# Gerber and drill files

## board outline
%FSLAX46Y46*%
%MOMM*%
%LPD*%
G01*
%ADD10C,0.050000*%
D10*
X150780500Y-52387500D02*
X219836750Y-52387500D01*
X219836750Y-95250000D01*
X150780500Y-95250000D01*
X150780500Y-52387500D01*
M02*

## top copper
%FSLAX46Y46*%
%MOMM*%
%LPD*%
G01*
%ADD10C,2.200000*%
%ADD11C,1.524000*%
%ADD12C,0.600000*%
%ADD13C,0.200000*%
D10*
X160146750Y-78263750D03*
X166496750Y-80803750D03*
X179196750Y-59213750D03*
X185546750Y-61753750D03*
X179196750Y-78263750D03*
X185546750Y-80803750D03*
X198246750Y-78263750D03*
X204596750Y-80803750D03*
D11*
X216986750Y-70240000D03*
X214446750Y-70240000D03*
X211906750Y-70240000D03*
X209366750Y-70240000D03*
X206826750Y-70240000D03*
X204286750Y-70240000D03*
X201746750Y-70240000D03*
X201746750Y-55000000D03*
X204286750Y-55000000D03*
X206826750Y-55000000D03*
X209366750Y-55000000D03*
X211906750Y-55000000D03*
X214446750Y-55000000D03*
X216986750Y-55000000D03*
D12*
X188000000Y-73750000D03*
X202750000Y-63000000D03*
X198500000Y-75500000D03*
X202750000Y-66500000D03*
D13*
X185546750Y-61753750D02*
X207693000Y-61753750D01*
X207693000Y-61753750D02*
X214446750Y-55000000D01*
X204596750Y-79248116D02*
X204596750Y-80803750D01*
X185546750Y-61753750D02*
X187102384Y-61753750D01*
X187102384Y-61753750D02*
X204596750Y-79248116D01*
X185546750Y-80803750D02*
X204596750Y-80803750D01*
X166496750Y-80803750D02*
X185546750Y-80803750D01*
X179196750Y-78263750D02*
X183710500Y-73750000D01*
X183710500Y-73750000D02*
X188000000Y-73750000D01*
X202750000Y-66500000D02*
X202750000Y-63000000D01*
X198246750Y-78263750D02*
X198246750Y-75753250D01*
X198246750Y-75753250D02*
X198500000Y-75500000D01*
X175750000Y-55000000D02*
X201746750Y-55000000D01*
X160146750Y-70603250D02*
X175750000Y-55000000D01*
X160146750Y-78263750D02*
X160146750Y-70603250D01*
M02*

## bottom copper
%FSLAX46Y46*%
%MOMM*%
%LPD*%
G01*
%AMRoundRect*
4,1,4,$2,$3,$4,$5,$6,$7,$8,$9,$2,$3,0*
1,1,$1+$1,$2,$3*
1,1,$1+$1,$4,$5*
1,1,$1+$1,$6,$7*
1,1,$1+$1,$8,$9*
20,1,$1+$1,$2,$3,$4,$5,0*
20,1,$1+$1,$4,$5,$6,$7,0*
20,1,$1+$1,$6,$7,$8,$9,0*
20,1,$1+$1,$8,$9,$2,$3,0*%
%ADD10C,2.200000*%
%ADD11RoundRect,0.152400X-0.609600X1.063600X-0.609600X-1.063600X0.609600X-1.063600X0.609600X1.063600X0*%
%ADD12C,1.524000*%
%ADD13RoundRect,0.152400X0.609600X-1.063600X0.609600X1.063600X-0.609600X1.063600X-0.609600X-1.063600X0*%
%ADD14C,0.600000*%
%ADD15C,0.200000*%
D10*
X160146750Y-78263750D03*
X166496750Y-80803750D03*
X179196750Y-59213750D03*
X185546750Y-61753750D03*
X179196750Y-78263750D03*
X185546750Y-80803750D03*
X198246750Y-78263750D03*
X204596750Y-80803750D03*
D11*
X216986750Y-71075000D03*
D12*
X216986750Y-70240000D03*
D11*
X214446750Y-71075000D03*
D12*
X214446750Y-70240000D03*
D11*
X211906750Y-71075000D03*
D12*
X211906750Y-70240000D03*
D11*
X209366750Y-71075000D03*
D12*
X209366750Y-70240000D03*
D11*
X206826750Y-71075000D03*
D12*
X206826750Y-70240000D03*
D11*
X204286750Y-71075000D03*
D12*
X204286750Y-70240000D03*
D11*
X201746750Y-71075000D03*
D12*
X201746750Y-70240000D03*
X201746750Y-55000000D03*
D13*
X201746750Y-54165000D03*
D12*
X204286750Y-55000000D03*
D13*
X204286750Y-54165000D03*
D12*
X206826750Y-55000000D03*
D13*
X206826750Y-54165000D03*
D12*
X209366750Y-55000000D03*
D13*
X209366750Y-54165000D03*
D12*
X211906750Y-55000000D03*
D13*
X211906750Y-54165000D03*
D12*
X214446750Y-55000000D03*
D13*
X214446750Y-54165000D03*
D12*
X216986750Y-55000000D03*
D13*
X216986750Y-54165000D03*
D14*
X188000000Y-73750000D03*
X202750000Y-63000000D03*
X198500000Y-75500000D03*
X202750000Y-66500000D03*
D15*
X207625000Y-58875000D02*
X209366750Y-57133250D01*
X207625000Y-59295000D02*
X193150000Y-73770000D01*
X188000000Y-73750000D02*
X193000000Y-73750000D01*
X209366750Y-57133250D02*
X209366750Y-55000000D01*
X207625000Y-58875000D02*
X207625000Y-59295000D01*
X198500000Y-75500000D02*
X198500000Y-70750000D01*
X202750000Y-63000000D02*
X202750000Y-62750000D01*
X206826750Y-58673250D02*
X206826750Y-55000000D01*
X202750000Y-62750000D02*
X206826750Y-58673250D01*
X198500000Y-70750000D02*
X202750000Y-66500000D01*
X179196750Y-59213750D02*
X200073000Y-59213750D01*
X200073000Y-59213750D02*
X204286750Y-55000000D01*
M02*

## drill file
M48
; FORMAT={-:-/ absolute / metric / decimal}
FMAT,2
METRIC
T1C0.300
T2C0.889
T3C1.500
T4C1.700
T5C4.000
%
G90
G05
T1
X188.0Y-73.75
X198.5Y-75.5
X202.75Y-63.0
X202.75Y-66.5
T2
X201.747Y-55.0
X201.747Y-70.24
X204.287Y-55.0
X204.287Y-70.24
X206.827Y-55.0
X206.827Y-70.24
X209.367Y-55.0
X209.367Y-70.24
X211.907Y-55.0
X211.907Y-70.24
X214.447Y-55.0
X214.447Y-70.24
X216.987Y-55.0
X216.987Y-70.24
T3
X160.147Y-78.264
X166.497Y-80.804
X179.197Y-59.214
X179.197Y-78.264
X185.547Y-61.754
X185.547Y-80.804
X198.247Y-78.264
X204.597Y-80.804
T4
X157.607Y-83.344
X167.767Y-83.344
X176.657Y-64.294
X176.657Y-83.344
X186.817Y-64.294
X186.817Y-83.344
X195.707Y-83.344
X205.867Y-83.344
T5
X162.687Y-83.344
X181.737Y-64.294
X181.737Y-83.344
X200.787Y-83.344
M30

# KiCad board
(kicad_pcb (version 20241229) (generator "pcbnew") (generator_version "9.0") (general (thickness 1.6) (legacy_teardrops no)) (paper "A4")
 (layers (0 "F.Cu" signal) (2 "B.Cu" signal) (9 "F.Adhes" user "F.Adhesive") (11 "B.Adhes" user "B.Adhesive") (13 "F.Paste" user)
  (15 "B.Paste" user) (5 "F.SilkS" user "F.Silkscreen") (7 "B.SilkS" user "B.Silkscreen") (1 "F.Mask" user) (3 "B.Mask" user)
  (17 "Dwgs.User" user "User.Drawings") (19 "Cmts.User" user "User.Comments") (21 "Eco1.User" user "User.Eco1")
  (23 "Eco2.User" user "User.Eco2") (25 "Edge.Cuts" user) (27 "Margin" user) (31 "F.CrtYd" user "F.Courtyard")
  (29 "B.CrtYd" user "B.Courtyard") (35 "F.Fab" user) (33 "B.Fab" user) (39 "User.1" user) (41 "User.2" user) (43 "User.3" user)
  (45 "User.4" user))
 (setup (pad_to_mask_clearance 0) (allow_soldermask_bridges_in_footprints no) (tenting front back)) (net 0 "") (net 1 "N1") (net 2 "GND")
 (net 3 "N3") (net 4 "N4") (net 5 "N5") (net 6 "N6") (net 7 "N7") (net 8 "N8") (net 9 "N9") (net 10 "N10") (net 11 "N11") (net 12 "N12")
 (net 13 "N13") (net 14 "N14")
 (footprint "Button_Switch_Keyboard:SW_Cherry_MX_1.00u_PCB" (layer "B.Cu") (at 160.14675 78.26375 180)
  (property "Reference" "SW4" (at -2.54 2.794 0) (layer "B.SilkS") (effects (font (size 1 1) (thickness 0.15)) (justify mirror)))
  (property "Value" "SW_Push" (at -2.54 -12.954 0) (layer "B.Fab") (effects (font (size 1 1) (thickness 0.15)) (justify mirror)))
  (pad "" np_thru_hole circle (at -7.62 -5.08 180) (size 1.7 1.7) (drill 1.7) (layers "*.Cu" "*.Mask"))
  (pad "" np_thru_hole circle (at -2.54 -5.08 180) (size 4 4) (drill 4) (layers "*.Cu" "*.Mask"))
  (pad "" np_thru_hole circle (at 2.54 -5.08 180) (size 1.7 1.7) (drill 1.7) (layers "*.Cu" "*.Mask"))
  (pad "1" thru_hole circle (at 0 0 180) (size 2.2 2.2) (drill 1.5) (layers "*.Cu" "*.Mask") (remove_unused_layers no) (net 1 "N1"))
  (pad "2" thru_hole circle (at -6.35 -2.54 180) (size 2.2 2.2) (drill 1.5) (layers "*.Cu" "*.Mask") (remove_unused_layers no) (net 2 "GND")))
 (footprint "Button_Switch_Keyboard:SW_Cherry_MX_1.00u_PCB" (layer "B.Cu") (at 179.19675 59.21375 180)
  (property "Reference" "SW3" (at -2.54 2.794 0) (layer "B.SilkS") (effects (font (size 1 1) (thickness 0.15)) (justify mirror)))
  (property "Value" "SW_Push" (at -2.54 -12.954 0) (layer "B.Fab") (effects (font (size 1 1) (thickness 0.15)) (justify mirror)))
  (pad "" np_thru_hole circle (at -7.62 -5.08 180) (size 1.7 1.7) (drill 1.7) (layers "*.Cu" "*.Mask"))
  (pad "" np_thru_hole circle (at -2.54 -5.08 180) (size 4 4) (drill 4) (layers "*.Cu" "*.Mask"))
  (pad "" np_thru_hole circle (at 2.54 -5.08 180) (size 1.7 1.7) (drill 1.7) (layers "*.Cu" "*.Mask"))
  (pad "1" thru_hole circle (at 0 0 180) (size 2.2 2.2) (drill 1.5) (layers "*.Cu" "*.Mask") (remove_unused_layers no) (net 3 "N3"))
  (pad "2" thru_hole circle (at -6.35 -2.54 180) (size 2.2 2.2) (drill 1.5) (layers "*.Cu" "*.Mask") (remove_unused_layers no) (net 2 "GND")))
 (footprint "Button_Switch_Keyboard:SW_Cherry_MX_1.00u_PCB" (layer "B.Cu") (at 179.19675 78.26375 180)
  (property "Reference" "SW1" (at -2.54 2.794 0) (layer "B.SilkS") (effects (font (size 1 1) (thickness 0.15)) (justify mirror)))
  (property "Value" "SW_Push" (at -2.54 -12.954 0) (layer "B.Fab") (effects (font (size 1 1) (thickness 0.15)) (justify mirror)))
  (pad "" np_thru_hole circle (at -7.62 -5.08 180) (size 1.7 1.7) (drill 1.7) (layers "*.Cu" "*.Mask"))
  (pad "" np_thru_hole circle (at -2.54 -5.08 180) (size 4 4) (drill 4) (layers "*.Cu" "*.Mask"))
  (pad "" np_thru_hole circle (at 2.54 -5.08 180) (size 1.7 1.7) (drill 1.7) (layers "*.Cu" "*.Mask"))
  (pad "1" thru_hole circle (at 0 0 180) (size 2.2 2.2) (drill 1.5) (layers "*.Cu" "*.Mask") (remove_unused_layers no) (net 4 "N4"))
  (pad "2" thru_hole circle (at -6.35 -2.54 180) (size 2.2 2.2) (drill 1.5) (layers "*.Cu" "*.Mask") (remove_unused_layers no) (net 2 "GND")))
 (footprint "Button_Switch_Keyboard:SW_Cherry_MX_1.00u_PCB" (layer "B.Cu") (at 198.24675 78.26375 180)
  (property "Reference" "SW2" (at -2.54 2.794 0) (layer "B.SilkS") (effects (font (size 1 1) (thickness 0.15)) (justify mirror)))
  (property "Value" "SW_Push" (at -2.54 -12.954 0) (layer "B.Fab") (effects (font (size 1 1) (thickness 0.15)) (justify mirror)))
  (pad "" np_thru_hole circle (at -7.62 -5.08 180) (size 1.7 1.7) (drill 1.7) (layers "*.Cu" "*.Mask"))
  (pad "" np_thru_hole circle (at -2.54 -5.08 180) (size 4 4) (drill 4) (layers "*.Cu" "*.Mask"))
  (pad "" np_thru_hole circle (at 2.54 -5.08 180) (size 1.7 1.7) (drill 1.7) (layers "*.Cu" "*.Mask"))
  (pad "1" thru_hole circle (at 0 0 180) (size 2.2 2.2) (drill 1.5) (layers "*.Cu" "*.Mask") (remove_unused_layers no) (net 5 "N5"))
  (pad "2" thru_hole circle (at -6.35 -2.54 180) (size 2.2 2.2) (drill 1.5) (layers "*.Cu" "*.Mask") (remove_unused_layers no) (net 2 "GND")))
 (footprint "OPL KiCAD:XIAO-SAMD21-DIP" (layer "B.Cu") (at 209.42925 62.52 90)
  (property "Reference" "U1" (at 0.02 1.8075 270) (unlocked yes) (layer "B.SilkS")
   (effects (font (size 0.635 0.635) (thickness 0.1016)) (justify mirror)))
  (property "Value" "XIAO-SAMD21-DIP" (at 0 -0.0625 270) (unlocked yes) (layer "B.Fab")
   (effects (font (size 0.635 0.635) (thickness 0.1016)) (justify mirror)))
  (pad "1" smd roundrect (at -8.555 7.5575 270) (size 2.432 1.524) (layers "B.Cu" "B.Mask") (roundrect_rratio 0.1) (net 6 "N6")
   (thermal_bridge_angle 45))
  (pad "1" thru_hole circle (at -7.72 7.5575 270) (size 1.524 1.524) (drill 0.889) (layers "*.Cu" "*.Mask") (remove_unused_layers no)
   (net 6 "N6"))
  (pad "2" smd roundrect (at -8.555 5.0175 270) (size 2.432 1.524) (layers "B.Cu" "B.Mask") (roundrect_rratio 0.1) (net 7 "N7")
   (thermal_bridge_angle 45))
  (pad "2" thru_hole circle (at -7.72 5.0175 270) (size 1.524 1.524) (drill 0.889) (layers "*.Cu" "*.Mask") (remove_unused_layers no)
   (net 7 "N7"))
  (pad "3" smd roundrect (at -8.555 2.4775 270) (size 2.432 1.524) (layers "B.Cu" "B.Mask") (roundrect_rratio 0.1) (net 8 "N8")
   (thermal_bridge_angle 45))
  (pad "3" thru_hole circle (at -7.72 2.4775 270) (size 1.524 1.524) (drill 0.889) (layers "*.Cu" "*.Mask") (remove_unused_layers no)
   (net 8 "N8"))
  (pad "4" smd roundrect (at -8.555 -0.0625 270) (size 2.432 1.524) (layers "B.Cu" "B.Mask") (roundrect_rratio 0.1) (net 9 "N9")
   (thermal_bridge_angle 45))
  (pad "4" thru_hole circle (at -7.72 -0.0625 270) (size 1.524 1.524) (drill 0.889) (layers "*.Cu" "*.Mask") (remove_unused_layers no)
   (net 9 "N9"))
  (pad "5" smd roundrect (at -8.555 -2.6025 270) (size 2.432 1.524) (layers "B.Cu" "B.Mask") (roundrect_rratio 0.1) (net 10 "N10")
   (thermal_bridge_angle 45))
  (pad "5" thru_hole circle (at -7.72 -2.6025 270) (size 1.524 1.524) (drill 0.889) (layers "*.Cu" "*.Mask") (remove_unused_layers no)
   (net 10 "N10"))
  (pad "6" smd roundrect (at -8.555 -5.1425 270) (size 2.432 1.524) (layers "B.Cu" "B.Mask") (roundrect_rratio 0.1) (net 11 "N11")
   (thermal_bridge_angle 45))
  (pad "6" thru_hole circle (at -7.72 -5.1425 270) (size 1.524 1.524) (drill 0.889) (layers "*.Cu" "*.Mask") (remove_unused_layers no)
   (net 11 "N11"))
  (pad "7" smd roundrect (at -8.555 -7.6825 270) (size 2.432 1.524) (layers "B.Cu" "B.Mask") (roundrect_rratio 0.1) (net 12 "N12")
   (thermal_bridge_angle 45))
  (pad "7" thru_hole circle (at -7.72 -7.6825 270) (size 1.524 1.524) (drill 0.889) (layers "*.Cu" "*.Mask") (remove_unused_layers no)
   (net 12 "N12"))
  (pad "8" thru_hole circle (at 7.52 -7.6825 90) (size 1.524 1.524) (drill 0.889) (layers "*.Cu" "*.Mask") (remove_unused_layers no)
   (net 1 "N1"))
  (pad "8" smd roundrect (at 8.355 -7.6825 90) (size 2.432 1.524) (layers "B.Cu" "B.Mask") (roundrect_rratio 0.1) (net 1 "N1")
   (thermal_bridge_angle 45))
  (pad "9" thru_hole circle (at 7.52 -5.1425 90) (size 1.524 1.524) (drill 0.889) (layers "*.Cu" "*.Mask") (remove_unused_layers no)
   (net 3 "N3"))
  (pad "9" smd roundrect (at 8.355 -5.1425 90) (size 2.432 1.524) (layers "B.Cu" "B.Mask") (roundrect_rratio 0.1) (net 3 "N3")
   (thermal_bridge_angle 45))
  (pad "10" thru_hole circle (at 7.52 -2.6025 90) (size 1.524 1.524) (drill 0.889) (layers "*.Cu" "*.Mask") (remove_unused_layers no)
   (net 5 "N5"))
  (pad "10" smd roundrect (at 8.355 -2.6025 90) (size 2.432 1.524) (layers "B.Cu" "B.Mask") (roundrect_rratio 0.1) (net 5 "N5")
   (thermal_bridge_angle 45))
  (pad "11" thru_hole circle (at 7.52 -0.0625 90) (size 1.524 1.524) (drill 0.889) (layers "*.Cu" "*.Mask") (remove_unused_layers no)
   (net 4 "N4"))
  (pad "11" smd roundrect (at 8.355 -0.0625 90) (size 2.432 1.524) (layers "B.Cu" "B.Mask") (roundrect_rratio 0.1) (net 4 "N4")
   (thermal_bridge_angle 45))
  (pad "12" thru_hole circle (at 7.52 2.4775 90) (size 1.524 1.524) (drill 0.889) (layers "*.Cu" "*.Mask") (remove_unused_layers no)
   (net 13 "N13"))
  (pad "12" smd roundrect (at 8.355 2.4775 90) (size 2.432 1.524) (layers "B.Cu" "B.Mask") (roundrect_rratio 0.1) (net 13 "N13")
   (thermal_bridge_angle 45))
  (pad "13" thru_hole circle (at 7.52 5.0175 90) (size 1.524 1.524) (drill 0.889) (layers "*.Cu" "*.Mask") (remove_unused_layers no)
   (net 2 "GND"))
  (pad "13" smd roundrect (at 8.355 5.0175 90) (size 2.432 1.524) (layers "B.Cu" "B.Mask") (roundrect_rratio 0.1) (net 2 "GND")
   (thermal_bridge_angle 45))
  (pad "14" thru_hole circle (at 7.52 7.5575 90) (size 1.524 1.524) (drill 0.889) (layers "*.Cu" "*.Mask") (remove_unused_layers no)
   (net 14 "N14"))
  (pad "14" smd roundrect (at 8.355 7.5575 90) (size 2.432 1.524) (layers "B.Cu" "B.Mask") (roundrect_rratio 0.1) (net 14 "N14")
   (thermal_bridge_angle 45)))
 (gr_rect (start 150.7805 52.3875) (end 219.83675 95.25) (stroke (width 0.05) (type default)) (fill no) (layer "Edge.Cuts"))
 (segment (start 185.54675 61.75375) (end 207.693 61.75375) (width 0.2) (layer "F.Cu") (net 2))
 (segment (start 207.693 61.75375) (end 214.44675 55) (width 0.2) (layer "F.Cu") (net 2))
 (segment (start 204.59675 79.248116) (end 204.59675 80.80375) (width 0.2) (layer "F.Cu") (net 2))
 (segment (start 185.54675 61.75375) (end 187.102384 61.75375) (width 0.2) (layer "F.Cu") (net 2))
 (segment (start 187.102384 61.75375) (end 204.59675 79.248116) (width 0.2) (layer "F.Cu") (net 2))
 (segment (start 185.54675 80.80375) (end 204.59675 80.80375) (width 0.2) (layer "F.Cu") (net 2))
 (segment (start 166.49675 80.80375) (end 185.54675 80.80375) (width 0.2) (layer "F.Cu") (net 2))
 (segment (start 179.19675 78.26375) (end 183.7105 73.75) (width 0.2) (layer "F.Cu") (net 4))
 (segment (start 183.7105 73.75) (end 188 73.75) (width 0.2) (layer "F.Cu") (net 4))
 (via (at 188 73.75) (size 0.6) (drill 0.3) (layers "F.Cu" "B.Cu") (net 4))
 (segment (start 207.625 58.875) (end 209.36675 57.13325) (width 0.2) (layer "B.Cu") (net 4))
 (segment (start 207.625 59.295) (end 193.15 73.77) (width 0.2) (layer "B.Cu") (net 4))
 (segment (start 188 73.75) (end 193 73.75) (width 0.2) (layer "B.Cu") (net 4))
 (segment (start 209.36675 57.13325) (end 209.36675 55) (width 0.2) (layer "B.Cu") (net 4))
 (segment (start 207.625 58.875) (end 207.625 59.295) (width 0.2) (layer "B.Cu") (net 4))
 (segment (start 202.75 66.5) (end 202.75 63) (width 0.2) (layer "F.Cu") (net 5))
 (segment (start 198.24675 78.26375) (end 198.24675 75.75325) (width 0.2) (layer "F.Cu") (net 5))
 (segment (start 198.24675 75.75325) (end 198.5 75.5) (width 0.2) (layer "F.Cu") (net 5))
 (via (at 202.75 63) (size 0.6) (drill 0.3) (layers "F.Cu" "B.Cu") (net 5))
 (via (at 198.5 75.5) (size 0.6) (drill 0.3) (layers "F.Cu" "B.Cu") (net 5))
 (via (at 202.75 66.5) (size 0.6) (drill 0.3) (layers "F.Cu" "B.Cu") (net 5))
 (segment (start 198.5 75.5) (end 198.5 70.75) (width 0.2) (layer "B.Cu") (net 5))
 (segment (start 202.75 63) (end 202.75 62.75) (width 0.2) (layer "B.Cu") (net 5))
 (segment (start 206.82675 58.67325) (end 206.82675 55) (width 0.2) (layer "B.Cu") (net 5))
 (segment (start 202.75 62.75) (end 206.82675 58.67325) (width 0.2) (layer "B.Cu") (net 5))
 (segment (start 198.5 70.75) (end 202.75 66.5) (width 0.2) (layer "B.Cu") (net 5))
 (segment (start 179.19675 59.21375) (end 200.073 59.21375) (width 0.2) (layer "B.Cu") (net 3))
 (segment (start 200.073 59.21375) (end 204.28675 55) (width 0.2) (layer "B.Cu") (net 3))
 (segment (start 175.75 55) (end 201.74675 55) (width 0.2) (layer "F.Cu") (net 1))
 (segment (start 160.14675 70.60325) (end 175.75 55) (width 0.2) (layer "F.Cu") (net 1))
 (segment (start 160.14675 78.26375) (end 160.14675 70.60325) (width 0.2) (layer "F.Cu") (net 1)))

